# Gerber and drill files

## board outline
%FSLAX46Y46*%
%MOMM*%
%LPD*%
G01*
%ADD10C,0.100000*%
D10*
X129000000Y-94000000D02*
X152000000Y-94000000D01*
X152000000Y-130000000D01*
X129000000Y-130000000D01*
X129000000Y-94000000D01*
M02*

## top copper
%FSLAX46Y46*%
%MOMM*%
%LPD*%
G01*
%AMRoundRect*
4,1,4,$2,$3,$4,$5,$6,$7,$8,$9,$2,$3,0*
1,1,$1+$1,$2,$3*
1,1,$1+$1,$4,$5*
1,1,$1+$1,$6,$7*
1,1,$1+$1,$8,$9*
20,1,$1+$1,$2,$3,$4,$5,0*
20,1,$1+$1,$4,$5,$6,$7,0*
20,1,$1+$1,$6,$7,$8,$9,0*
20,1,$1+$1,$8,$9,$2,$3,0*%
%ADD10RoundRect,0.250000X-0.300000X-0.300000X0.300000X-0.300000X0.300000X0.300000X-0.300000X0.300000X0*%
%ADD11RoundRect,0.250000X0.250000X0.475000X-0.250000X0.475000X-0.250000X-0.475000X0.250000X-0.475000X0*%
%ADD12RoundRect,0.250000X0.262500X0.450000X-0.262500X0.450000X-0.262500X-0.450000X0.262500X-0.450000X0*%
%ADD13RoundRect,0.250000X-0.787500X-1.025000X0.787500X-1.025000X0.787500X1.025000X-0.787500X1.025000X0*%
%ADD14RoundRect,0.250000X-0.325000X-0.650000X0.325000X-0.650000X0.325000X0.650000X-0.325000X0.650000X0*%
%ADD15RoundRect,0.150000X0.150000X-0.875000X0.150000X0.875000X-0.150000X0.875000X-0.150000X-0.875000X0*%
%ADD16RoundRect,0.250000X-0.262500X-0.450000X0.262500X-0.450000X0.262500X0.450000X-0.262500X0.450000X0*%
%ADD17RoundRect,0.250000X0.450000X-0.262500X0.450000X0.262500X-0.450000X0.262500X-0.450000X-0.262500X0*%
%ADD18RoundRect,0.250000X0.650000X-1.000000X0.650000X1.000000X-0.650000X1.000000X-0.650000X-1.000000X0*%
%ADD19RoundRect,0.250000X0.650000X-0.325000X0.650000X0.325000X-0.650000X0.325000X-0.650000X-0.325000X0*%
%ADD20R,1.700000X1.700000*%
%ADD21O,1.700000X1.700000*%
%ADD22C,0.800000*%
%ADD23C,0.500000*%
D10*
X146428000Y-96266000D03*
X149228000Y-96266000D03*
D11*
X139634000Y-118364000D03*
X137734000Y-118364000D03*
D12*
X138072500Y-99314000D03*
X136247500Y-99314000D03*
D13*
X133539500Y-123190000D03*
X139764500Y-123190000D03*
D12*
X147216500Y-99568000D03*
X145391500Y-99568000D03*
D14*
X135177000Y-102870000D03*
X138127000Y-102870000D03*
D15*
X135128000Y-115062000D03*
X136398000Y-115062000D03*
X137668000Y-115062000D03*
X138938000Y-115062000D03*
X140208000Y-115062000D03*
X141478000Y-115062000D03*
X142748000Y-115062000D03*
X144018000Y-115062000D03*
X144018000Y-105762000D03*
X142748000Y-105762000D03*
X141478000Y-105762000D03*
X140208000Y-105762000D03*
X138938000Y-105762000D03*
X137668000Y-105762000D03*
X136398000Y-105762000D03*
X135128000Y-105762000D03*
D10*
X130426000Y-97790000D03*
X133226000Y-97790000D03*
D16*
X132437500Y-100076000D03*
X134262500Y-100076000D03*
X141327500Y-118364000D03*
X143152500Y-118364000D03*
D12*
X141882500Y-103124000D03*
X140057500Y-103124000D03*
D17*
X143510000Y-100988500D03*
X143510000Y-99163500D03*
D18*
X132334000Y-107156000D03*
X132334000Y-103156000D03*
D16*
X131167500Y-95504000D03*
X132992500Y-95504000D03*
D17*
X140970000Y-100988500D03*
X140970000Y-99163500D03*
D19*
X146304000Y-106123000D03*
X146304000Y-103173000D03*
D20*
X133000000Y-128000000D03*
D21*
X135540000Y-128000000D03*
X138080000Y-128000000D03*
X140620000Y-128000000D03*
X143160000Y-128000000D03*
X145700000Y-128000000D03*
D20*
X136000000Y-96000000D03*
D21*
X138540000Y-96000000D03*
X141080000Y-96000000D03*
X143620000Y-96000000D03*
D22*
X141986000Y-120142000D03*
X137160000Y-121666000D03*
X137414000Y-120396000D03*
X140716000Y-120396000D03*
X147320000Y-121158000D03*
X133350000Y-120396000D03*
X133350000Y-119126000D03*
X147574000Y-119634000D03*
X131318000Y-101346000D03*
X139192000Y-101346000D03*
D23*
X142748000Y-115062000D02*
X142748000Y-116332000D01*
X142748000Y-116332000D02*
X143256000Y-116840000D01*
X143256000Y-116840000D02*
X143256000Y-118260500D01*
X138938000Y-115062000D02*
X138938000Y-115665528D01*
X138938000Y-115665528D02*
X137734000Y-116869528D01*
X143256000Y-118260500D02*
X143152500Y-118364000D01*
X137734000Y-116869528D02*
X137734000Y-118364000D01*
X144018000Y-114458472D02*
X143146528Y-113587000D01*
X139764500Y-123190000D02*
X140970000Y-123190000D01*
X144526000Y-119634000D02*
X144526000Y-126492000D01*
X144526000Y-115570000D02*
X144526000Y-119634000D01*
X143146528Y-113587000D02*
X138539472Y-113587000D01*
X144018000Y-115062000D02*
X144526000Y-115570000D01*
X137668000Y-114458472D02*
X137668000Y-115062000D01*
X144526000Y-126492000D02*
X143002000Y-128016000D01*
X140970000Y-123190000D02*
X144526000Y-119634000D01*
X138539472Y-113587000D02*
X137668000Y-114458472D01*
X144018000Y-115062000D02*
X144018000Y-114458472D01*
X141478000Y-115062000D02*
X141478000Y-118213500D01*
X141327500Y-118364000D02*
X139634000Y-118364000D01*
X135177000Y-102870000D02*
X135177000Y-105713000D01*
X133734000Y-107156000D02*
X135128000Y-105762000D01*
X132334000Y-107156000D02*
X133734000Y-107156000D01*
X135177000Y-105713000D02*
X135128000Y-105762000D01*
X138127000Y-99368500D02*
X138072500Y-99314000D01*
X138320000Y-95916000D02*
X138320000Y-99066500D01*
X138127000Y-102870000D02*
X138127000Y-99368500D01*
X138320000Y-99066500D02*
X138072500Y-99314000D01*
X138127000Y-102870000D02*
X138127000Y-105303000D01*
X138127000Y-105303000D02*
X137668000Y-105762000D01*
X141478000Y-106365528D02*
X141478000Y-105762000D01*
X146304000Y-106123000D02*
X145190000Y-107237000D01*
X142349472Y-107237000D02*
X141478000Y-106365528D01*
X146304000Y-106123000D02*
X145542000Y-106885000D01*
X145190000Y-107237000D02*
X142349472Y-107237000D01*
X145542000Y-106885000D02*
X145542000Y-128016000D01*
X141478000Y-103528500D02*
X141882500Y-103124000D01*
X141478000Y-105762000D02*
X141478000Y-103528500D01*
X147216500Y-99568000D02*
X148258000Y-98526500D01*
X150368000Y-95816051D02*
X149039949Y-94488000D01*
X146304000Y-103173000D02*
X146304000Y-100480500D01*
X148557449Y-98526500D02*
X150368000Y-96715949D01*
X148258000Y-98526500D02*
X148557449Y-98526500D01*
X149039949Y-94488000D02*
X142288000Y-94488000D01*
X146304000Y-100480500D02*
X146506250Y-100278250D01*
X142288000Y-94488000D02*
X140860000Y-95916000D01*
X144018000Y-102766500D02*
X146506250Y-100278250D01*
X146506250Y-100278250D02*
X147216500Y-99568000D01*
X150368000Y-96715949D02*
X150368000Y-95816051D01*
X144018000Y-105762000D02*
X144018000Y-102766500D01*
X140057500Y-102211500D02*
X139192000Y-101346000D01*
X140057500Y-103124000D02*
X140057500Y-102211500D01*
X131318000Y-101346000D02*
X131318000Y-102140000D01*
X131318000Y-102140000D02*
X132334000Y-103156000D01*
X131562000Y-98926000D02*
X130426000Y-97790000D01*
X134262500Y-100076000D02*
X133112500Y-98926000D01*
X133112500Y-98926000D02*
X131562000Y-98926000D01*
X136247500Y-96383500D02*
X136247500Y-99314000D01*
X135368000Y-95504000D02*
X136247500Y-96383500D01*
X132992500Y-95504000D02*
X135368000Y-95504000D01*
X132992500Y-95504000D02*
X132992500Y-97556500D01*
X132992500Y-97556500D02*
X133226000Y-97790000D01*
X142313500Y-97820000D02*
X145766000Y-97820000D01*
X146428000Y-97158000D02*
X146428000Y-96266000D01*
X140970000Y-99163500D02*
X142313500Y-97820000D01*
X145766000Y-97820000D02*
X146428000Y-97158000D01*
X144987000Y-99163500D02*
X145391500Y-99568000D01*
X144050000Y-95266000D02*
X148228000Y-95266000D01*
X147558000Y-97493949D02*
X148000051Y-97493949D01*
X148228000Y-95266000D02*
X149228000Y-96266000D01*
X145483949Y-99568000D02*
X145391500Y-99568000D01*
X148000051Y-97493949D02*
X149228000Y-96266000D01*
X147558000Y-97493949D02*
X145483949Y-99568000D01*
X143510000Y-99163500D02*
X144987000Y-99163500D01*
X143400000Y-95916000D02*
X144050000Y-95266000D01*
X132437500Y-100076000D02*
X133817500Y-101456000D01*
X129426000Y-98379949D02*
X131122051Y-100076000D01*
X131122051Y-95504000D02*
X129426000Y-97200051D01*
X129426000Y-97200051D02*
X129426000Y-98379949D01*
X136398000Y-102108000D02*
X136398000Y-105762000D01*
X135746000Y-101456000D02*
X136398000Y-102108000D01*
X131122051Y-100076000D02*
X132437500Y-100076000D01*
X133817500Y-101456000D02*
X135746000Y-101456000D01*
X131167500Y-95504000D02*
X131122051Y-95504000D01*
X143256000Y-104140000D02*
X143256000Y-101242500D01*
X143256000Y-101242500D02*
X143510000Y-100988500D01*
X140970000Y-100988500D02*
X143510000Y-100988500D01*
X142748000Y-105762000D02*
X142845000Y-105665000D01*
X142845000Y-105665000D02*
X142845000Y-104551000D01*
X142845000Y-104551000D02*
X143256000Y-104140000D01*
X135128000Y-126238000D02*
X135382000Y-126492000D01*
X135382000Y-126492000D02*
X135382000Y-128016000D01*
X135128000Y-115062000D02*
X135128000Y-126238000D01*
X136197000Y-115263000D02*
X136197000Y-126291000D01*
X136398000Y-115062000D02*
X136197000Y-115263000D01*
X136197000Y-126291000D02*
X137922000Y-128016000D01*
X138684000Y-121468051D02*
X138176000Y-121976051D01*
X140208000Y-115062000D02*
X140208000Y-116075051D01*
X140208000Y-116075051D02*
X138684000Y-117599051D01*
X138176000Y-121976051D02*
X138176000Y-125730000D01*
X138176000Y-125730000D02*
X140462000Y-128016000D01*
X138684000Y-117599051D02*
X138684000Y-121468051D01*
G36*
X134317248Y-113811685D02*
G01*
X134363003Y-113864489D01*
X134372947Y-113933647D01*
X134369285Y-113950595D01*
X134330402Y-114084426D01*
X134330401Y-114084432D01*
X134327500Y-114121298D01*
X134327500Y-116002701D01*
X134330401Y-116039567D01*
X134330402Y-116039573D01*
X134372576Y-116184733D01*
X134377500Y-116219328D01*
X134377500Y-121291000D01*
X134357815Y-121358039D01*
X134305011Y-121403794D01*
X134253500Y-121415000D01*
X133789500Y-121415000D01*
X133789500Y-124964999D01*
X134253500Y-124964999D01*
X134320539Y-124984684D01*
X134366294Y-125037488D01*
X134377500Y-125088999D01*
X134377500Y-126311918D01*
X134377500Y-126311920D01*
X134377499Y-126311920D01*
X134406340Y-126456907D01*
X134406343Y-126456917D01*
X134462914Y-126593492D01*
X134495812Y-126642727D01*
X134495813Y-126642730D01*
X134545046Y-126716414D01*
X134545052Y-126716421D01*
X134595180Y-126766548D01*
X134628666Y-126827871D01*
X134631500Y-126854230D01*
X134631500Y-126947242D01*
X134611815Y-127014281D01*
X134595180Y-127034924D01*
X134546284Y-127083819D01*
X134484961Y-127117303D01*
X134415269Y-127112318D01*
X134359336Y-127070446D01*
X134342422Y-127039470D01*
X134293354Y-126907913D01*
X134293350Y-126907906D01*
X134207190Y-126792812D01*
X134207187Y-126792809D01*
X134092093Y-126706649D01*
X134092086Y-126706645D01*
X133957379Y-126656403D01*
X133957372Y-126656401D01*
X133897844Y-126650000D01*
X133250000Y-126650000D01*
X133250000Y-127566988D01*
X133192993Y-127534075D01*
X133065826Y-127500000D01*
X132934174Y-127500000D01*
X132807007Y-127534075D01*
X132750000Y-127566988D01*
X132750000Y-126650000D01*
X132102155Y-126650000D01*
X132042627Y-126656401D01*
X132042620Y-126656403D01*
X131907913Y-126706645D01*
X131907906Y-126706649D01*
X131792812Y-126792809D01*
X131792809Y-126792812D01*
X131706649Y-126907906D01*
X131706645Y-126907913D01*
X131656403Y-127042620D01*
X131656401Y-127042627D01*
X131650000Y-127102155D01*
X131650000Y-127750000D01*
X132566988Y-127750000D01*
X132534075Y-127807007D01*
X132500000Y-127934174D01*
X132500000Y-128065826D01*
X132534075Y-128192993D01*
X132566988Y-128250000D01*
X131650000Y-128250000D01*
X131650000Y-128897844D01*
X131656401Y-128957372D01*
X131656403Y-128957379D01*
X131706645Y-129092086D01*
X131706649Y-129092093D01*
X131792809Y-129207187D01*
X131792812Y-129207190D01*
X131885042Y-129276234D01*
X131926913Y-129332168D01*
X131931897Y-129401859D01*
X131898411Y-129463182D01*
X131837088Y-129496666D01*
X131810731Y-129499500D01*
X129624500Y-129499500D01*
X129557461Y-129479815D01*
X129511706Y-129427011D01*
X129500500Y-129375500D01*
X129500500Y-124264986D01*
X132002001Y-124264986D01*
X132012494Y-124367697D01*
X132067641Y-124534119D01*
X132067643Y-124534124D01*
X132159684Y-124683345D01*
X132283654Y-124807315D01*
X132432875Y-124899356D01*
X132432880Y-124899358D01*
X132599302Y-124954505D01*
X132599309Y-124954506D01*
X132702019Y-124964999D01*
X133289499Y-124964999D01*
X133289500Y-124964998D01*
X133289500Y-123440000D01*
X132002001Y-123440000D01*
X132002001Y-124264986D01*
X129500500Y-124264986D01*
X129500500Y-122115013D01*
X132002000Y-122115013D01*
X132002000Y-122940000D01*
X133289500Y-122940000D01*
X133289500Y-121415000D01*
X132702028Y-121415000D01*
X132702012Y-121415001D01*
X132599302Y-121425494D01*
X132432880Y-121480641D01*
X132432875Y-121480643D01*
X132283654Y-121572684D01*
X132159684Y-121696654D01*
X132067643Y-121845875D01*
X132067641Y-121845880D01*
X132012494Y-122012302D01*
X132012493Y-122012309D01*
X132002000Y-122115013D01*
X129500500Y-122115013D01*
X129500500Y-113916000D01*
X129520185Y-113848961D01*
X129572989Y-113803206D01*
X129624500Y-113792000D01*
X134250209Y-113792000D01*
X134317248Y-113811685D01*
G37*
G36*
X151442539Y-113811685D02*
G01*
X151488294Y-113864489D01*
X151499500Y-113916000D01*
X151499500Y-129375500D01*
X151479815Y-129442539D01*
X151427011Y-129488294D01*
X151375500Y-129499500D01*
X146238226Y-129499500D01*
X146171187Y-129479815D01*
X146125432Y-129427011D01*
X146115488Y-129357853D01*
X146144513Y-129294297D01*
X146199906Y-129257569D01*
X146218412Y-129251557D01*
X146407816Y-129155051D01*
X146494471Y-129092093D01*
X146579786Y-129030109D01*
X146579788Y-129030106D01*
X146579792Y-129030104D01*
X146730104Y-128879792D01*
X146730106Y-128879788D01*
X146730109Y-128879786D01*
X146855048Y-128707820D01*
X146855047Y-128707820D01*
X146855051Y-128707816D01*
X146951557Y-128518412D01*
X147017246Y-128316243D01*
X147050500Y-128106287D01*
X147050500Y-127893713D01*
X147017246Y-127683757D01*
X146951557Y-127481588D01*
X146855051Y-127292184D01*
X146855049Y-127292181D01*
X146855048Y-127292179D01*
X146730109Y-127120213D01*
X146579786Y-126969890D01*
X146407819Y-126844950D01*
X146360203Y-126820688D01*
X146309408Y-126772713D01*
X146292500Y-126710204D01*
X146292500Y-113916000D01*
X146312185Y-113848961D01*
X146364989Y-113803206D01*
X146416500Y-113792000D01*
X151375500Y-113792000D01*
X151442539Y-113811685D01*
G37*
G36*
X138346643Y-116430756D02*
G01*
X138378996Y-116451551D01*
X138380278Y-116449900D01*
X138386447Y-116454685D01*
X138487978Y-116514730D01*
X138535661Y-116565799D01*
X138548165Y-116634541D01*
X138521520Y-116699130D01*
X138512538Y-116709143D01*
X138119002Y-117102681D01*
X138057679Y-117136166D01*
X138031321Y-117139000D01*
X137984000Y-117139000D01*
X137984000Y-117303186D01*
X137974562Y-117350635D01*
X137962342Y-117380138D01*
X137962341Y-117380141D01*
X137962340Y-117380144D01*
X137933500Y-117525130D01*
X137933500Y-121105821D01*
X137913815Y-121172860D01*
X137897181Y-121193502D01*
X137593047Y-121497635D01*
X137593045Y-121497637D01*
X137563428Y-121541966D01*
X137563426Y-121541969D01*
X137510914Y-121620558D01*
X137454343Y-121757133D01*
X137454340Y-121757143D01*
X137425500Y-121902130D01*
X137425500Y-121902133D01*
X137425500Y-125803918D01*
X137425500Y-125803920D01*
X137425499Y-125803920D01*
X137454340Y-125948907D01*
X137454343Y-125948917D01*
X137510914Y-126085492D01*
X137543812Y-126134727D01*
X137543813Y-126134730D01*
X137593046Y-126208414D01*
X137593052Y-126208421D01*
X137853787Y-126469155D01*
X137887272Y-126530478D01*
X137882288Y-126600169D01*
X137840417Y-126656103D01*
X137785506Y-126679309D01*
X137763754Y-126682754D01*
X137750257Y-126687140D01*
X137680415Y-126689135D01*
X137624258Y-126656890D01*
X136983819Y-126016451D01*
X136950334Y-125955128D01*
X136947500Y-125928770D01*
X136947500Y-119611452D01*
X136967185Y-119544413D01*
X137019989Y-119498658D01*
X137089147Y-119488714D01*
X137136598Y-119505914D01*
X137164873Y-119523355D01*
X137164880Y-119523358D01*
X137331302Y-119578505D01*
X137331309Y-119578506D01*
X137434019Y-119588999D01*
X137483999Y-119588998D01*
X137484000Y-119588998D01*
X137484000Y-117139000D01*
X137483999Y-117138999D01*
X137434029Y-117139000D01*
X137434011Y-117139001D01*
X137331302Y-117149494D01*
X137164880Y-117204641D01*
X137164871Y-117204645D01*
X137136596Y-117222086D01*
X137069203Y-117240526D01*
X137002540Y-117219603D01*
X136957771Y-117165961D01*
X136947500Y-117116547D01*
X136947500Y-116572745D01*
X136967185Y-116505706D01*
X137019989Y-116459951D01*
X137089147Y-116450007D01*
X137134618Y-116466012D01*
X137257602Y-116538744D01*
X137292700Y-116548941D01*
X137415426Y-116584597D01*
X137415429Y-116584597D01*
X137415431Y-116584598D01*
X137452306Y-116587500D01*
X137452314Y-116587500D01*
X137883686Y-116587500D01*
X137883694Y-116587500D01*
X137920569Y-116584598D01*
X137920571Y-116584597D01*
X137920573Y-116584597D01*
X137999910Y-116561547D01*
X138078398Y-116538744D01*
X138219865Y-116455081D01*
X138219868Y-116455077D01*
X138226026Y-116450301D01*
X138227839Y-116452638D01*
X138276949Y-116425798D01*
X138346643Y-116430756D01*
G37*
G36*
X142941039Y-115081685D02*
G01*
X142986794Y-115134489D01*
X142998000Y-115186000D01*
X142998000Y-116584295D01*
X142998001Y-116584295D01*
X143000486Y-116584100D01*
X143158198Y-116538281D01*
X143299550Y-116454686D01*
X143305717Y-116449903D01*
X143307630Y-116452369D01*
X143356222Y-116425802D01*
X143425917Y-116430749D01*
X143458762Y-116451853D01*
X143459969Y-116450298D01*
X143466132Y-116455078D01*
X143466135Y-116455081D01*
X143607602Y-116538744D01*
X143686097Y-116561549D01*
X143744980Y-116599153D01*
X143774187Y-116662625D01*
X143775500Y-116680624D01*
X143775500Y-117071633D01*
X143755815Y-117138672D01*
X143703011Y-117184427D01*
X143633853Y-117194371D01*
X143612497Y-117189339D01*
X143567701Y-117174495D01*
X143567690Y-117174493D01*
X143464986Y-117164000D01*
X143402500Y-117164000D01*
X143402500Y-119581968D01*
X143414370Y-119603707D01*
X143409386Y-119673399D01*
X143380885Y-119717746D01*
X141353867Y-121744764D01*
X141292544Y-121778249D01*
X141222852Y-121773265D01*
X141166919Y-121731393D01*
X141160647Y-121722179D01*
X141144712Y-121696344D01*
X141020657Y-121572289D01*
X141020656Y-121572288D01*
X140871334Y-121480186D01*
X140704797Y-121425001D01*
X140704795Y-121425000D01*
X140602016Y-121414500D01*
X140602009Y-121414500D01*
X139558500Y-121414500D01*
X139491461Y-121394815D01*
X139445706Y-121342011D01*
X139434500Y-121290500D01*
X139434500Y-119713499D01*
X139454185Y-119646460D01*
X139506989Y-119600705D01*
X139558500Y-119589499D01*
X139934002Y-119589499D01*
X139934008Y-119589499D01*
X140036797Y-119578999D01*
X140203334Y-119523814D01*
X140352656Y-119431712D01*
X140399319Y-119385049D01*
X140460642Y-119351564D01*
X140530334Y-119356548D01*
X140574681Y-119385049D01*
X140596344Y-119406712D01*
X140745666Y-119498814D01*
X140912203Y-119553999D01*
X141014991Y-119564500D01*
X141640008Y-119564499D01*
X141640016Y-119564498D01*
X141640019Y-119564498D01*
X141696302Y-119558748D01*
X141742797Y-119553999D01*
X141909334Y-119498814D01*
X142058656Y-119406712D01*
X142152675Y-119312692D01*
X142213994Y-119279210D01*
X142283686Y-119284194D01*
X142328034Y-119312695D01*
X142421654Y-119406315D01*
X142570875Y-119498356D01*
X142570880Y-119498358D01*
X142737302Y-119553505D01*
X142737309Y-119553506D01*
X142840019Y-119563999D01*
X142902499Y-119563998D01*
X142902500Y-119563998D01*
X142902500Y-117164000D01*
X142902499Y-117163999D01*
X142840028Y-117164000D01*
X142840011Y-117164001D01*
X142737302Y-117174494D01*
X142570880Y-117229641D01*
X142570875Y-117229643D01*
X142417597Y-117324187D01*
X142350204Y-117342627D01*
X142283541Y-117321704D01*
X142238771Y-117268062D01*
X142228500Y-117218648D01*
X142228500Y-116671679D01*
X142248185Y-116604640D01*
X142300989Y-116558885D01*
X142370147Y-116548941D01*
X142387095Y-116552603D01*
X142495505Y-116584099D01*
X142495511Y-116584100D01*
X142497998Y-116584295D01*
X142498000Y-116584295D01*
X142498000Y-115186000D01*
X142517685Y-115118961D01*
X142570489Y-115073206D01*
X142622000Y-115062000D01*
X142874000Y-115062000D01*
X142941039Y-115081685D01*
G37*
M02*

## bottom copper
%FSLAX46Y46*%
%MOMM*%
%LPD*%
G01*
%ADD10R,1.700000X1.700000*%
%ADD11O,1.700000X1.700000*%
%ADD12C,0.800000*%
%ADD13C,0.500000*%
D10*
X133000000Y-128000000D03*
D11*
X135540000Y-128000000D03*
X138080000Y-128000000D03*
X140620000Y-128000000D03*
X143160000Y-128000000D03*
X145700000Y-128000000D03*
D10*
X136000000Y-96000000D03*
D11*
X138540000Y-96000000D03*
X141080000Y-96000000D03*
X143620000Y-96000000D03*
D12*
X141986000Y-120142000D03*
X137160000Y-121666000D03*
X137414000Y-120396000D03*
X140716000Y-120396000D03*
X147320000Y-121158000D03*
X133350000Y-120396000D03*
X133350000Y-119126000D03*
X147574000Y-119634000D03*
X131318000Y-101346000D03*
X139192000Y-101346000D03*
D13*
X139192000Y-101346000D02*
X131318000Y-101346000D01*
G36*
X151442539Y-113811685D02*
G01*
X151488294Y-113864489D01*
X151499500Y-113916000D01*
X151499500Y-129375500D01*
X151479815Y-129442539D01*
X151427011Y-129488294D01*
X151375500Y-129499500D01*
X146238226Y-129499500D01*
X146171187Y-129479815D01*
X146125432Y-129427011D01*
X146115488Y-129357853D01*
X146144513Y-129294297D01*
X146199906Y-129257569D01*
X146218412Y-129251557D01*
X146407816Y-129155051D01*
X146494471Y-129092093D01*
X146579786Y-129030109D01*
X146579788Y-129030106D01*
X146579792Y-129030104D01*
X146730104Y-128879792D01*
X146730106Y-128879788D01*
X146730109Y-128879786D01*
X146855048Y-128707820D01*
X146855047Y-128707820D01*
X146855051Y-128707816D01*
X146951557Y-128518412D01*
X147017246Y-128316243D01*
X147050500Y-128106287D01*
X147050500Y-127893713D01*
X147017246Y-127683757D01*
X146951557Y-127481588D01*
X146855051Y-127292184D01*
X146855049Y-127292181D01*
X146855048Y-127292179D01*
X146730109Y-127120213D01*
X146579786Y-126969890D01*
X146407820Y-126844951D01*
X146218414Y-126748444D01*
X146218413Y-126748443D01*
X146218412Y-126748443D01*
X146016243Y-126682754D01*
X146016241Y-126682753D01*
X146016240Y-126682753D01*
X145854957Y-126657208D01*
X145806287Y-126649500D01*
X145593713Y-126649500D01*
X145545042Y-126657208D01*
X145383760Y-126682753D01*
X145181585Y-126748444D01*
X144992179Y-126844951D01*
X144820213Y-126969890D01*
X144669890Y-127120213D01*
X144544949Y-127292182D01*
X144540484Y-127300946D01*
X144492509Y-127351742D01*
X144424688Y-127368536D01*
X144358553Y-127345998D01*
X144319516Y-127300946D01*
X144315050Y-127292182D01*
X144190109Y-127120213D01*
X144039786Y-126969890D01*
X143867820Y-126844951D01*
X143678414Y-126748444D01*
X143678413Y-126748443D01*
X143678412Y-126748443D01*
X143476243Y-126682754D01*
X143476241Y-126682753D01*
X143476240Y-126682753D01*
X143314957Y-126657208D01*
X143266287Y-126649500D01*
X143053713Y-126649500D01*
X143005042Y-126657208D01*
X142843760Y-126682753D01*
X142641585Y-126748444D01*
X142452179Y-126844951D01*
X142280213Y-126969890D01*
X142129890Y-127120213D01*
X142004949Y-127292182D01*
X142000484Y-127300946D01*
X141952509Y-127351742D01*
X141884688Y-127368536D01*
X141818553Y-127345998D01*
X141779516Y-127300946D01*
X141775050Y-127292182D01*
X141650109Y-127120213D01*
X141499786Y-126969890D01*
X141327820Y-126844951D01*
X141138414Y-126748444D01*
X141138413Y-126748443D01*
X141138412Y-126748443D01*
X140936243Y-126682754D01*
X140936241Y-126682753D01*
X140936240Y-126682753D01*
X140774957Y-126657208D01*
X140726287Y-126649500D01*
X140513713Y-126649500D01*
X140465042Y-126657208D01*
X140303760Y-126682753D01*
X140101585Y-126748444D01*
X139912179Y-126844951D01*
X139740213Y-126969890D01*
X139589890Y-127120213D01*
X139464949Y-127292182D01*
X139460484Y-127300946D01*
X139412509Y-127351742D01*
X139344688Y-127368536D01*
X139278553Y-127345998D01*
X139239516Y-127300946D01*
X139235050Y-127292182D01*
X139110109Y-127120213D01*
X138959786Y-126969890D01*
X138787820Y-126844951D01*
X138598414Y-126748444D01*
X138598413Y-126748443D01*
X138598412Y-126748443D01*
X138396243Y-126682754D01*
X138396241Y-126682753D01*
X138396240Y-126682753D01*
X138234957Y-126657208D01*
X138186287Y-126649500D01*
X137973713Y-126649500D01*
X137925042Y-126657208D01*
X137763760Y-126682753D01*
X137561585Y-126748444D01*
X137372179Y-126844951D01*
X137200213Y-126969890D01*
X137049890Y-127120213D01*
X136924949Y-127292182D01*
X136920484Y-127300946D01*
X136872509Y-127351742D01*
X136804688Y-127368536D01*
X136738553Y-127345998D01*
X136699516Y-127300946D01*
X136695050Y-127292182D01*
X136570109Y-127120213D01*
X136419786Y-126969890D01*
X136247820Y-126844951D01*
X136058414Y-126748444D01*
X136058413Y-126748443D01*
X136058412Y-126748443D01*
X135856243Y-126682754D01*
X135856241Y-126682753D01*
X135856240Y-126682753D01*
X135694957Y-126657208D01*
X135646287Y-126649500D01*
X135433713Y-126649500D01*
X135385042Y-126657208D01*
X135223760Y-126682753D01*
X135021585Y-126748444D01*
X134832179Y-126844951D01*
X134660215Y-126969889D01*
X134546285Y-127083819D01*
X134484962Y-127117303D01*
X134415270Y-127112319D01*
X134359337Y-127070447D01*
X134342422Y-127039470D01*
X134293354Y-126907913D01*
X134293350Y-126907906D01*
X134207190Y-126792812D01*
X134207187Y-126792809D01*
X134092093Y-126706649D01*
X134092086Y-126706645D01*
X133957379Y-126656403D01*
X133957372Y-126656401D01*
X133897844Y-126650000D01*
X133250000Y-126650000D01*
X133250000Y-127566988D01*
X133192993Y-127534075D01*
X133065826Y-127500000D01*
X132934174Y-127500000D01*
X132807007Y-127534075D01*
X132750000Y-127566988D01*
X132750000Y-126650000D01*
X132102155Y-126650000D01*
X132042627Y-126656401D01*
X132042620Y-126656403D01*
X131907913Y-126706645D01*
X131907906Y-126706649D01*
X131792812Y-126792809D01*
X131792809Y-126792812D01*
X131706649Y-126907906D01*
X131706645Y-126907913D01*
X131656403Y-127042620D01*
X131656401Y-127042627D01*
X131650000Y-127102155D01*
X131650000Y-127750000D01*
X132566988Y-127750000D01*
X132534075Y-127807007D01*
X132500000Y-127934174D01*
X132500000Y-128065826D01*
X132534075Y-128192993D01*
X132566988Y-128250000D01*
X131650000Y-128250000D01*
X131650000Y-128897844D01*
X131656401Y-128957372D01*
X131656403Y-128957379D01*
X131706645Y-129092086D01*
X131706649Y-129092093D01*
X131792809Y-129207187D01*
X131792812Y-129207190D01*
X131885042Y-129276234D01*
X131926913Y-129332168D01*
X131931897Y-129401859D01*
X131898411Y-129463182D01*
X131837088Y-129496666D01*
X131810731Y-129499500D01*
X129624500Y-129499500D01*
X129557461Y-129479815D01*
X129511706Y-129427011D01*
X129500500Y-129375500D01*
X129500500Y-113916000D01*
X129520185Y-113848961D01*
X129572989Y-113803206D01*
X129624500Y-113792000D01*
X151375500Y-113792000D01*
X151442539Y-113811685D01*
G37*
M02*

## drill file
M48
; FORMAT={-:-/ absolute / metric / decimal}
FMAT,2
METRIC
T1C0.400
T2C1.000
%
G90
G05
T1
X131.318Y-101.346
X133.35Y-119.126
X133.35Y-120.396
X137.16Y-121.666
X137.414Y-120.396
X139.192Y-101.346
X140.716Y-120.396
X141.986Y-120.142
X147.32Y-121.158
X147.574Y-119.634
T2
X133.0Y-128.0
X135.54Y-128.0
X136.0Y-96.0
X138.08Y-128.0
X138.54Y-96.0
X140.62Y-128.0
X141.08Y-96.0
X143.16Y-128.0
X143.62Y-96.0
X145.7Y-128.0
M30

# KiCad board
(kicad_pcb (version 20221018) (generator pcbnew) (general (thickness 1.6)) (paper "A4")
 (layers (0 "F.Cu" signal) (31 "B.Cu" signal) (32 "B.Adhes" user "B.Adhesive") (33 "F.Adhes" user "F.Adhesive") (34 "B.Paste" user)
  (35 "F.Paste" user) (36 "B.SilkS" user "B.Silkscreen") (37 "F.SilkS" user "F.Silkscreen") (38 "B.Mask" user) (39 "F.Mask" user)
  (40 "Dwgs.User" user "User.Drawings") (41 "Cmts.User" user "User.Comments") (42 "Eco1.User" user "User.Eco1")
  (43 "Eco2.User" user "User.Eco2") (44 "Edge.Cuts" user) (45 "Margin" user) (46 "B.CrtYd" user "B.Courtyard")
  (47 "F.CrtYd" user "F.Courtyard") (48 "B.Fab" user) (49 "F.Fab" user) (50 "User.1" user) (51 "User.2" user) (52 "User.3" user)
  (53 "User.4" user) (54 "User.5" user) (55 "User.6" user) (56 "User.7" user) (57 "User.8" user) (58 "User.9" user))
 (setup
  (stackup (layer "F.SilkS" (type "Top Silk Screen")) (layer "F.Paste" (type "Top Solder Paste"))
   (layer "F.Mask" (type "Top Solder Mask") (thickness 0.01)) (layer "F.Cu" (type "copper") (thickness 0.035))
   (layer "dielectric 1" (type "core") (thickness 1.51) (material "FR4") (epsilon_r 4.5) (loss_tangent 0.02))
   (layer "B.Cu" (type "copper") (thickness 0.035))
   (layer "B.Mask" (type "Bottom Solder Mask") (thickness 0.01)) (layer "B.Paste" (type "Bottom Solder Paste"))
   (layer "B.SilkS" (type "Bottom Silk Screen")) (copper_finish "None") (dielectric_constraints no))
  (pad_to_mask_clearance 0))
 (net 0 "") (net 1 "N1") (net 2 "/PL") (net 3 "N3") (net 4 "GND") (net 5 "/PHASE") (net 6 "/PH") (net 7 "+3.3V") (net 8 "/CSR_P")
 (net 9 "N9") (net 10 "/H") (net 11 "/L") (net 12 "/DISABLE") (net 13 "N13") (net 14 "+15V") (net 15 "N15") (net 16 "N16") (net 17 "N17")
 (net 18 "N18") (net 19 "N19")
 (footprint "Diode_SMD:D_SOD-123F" (layer "F.Cu") (at 147.828 96.266)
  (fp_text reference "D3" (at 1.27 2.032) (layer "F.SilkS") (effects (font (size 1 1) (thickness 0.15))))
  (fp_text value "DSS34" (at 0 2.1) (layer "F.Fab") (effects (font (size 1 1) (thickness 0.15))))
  (pad "1" smd roundrect (at -1.4 0) (size 1.1 1.1) (layers "F.Cu" "F.Paste" "F.Mask") (roundrect_rratio 0.2272727273) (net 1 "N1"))
  (pad "2" smd roundrect (at 1.4 0) (size 1.1 1.1) (layers "F.Cu" "F.Paste" "F.Mask") (roundrect_rratio 0.2272727273) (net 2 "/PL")))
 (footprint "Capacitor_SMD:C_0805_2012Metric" (layer "F.Cu") (at 138.684 118.364 180)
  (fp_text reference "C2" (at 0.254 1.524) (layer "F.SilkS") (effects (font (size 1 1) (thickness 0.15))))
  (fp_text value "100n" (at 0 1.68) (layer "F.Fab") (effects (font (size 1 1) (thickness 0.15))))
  (pad "1" smd roundrect (at -0.95 0 180) (size 1 1.45) (layers "F.Cu" "F.Paste" "F.Mask") (roundrect_rratio 0.25) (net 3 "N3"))
  (pad "2" smd roundrect (at 0.95 0 180) (size 1 1.45) (layers "F.Cu" "F.Paste" "F.Mask") (roundrect_rratio 0.25) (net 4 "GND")))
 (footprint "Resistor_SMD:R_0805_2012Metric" (layer "F.Cu") (at 137.16 99.314 180)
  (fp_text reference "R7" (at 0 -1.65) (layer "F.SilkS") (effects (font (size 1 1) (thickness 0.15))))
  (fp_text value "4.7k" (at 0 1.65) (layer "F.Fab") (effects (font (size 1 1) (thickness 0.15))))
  (pad "1" smd roundrect (at -0.9125 0 180) (size 1.025 1.4) (layers "F.Cu" "F.Paste" "F.Mask") (roundrect_rratio 0.243902) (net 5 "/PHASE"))
  (pad "2" smd roundrect (at 0.9125 0 180) (size 1.025 1.4) (layers "F.Cu" "F.Paste" "F.Mask") (roundrect_rratio 0.243902) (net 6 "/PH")))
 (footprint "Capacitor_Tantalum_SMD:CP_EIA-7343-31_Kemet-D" (layer "F.Cu") (at 136.652 123.19)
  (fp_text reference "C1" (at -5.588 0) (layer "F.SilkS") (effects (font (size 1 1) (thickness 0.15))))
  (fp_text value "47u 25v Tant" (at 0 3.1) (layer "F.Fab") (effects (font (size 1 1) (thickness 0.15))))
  (pad "1" smd roundrect (at -3.1125 0) (size 2.075 2.55) (layers "F.Cu" "F.Paste" "F.Mask") (roundrect_rratio 0.120482) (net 4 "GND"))
  (pad "2" smd roundrect (at 3.1125 0) (size 2.075 2.55) (layers "F.Cu" "F.Paste" "F.Mask") (roundrect_rratio 0.120482) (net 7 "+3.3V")))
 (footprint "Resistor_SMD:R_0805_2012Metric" (layer "F.Cu") (at 146.304 99.568 180)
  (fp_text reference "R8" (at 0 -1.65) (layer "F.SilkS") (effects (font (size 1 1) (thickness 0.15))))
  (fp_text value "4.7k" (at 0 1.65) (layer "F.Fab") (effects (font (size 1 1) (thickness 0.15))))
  (pad "1" smd roundrect (at -0.9125 0 180) (size 1.025 1.4) (layers "F.Cu" "F.Paste" "F.Mask") (roundrect_rratio 0.243902) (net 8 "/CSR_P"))
  (pad "2" smd roundrect (at 0.9125 0 180) (size 1.025 1.4) (layers "F.Cu" "F.Paste" "F.Mask") (roundrect_rratio 0.243902) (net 2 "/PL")))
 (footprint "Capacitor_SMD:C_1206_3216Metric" (layer "F.Cu") (at 136.652 102.87)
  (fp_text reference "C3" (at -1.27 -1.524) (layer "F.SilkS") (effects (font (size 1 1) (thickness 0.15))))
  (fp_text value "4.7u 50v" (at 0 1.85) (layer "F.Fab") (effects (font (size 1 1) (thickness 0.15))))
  (pad "1" smd roundrect (at -1.475 0) (size 1.15 1.8) (layers "F.Cu" "F.Paste" "F.Mask") (roundrect_rratio 0.217391) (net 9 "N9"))
  (pad "2" smd roundrect (at 1.475 0) (size 1.15 1.8) (layers "F.Cu" "F.Paste" "F.Mask") (roundrect_rratio 0.217391) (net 5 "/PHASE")))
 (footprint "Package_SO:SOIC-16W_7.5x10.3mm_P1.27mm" (layer "F.Cu") (at 139.573 110.412 90)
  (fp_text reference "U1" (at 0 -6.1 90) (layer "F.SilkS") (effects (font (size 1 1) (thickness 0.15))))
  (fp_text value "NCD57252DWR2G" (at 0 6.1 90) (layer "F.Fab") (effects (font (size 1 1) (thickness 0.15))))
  (pad "1" smd roundrect (at -4.65 -4.445 90) (size 2.05 0.6) (layers "F.Cu" "F.Paste" "F.Mask") (roundrect_rratio 0.25) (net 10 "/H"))
  (pad "2" smd roundrect (at -4.65 -3.175 90) (size 2.05 0.6) (layers "F.Cu" "F.Paste" "F.Mask") (roundrect_rratio 0.25) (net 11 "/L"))
  (pad "3" smd roundrect (at -4.65 -1.905 90) (size 2.05 0.6) (layers "F.Cu" "F.Paste" "F.Mask") (roundrect_rratio 0.25) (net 7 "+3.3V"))
  (pad "4" smd roundrect (at -4.65 -0.635 90) (size 2.05 0.6) (layers "F.Cu" "F.Paste" "F.Mask") (roundrect_rratio 0.25) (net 4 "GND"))
  (pad "5" smd roundrect (at -4.65 0.635 90) (size 2.05 0.6) (layers "F.Cu" "F.Paste" "F.Mask") (roundrect_rratio 0.25) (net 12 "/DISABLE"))
  (pad "6" smd roundrect (at -4.65 1.905 90) (size 2.05 0.6) (layers "F.Cu" "F.Paste" "F.Mask") (roundrect_rratio 0.25) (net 3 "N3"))
  (pad "7" smd roundrect (at -4.65 3.175 90) (size 2.05 0.6) (layers "F.Cu" "F.Paste" "F.Mask") (roundrect_rratio 0.25) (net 4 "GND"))
  (pad "8" smd roundrect (at -4.65 4.445 90) (size 2.05 0.6) (layers "F.Cu" "F.Paste" "F.Mask") (roundrect_rratio 0.25) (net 7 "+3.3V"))
  (pad "9" smd roundrect (at 4.65 4.445 90) (size 2.05 0.6) (layers "F.Cu" "F.Paste" "F.Mask") (roundrect_rratio 0.25) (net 8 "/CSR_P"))
  (pad "10" smd roundrect (at 4.65 3.175 90) (size 2.05 0.6) (layers "F.Cu" "F.Paste" "F.Mask") (roundrect_rratio 0.25) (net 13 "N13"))
  (pad "11" smd roundrect (at 4.65 1.905 90) (size 2.05 0.6) (layers "F.Cu" "F.Paste" "F.Mask") (roundrect_rratio 0.25) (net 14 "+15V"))
  (pad "12" smd roundrect (at 4.65 0.635 90) (size 2.05 0.6) (layers "F.Cu" "F.Paste" "F.Mask") (roundrect_rratio 0.25) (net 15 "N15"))
  (pad "13" smd roundrect (at 4.65 -0.635 90) (size 2.05 0.6) (layers "F.Cu" "F.Paste" "F.Mask") (roundrect_rratio 0.25) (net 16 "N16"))
  (pad "14" smd roundrect (at 4.65 -1.905 90) (size 2.05 0.6) (layers "F.Cu" "F.Paste" "F.Mask") (roundrect_rratio 0.25) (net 5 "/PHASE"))
  (pad "15" smd roundrect (at 4.65 -3.175 90) (size 2.05 0.6) (layers "F.Cu" "F.Paste" "F.Mask") (roundrect_rratio 0.25) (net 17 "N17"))
  (pad "16" smd roundrect (at 4.65 -4.445 90) (size 2.05 0.6) (layers "F.Cu" "F.Paste" "F.Mask") (roundrect_rratio 0.25) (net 9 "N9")))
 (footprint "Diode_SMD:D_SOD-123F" (layer "F.Cu") (at 131.826 97.79)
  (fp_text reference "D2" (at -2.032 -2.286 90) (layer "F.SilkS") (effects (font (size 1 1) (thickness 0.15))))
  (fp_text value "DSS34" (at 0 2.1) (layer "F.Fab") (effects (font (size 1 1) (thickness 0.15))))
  (pad "1" smd roundrect (at -1.4 0) (size 1.1 1.1) (layers "F.Cu" "F.Paste" "F.Mask") (roundrect_rratio 0.2272727273) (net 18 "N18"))
  (pad "2" smd roundrect (at 1.4 0) (size 1.1 1.1) (layers "F.Cu" "F.Paste" "F.Mask") (roundrect_rratio 0.2272727273) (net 6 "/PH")))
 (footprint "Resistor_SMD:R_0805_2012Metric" (layer "F.Cu") (at 133.35 100.076)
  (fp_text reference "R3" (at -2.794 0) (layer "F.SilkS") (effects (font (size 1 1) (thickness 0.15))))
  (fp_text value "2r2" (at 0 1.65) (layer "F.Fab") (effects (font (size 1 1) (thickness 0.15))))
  (pad "1" smd roundrect (at -0.9125 0) (size 1.025 1.4) (layers "F.Cu" "F.Paste" "F.Mask") (roundrect_rratio 0.243902) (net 17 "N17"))
  (pad "2" smd roundrect (at 0.9125 0) (size 1.025 1.4) (layers "F.Cu" "F.Paste" "F.Mask") (roundrect_rratio 0.243902) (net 18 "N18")))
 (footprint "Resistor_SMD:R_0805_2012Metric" (layer "F.Cu") (at 142.24 118.364)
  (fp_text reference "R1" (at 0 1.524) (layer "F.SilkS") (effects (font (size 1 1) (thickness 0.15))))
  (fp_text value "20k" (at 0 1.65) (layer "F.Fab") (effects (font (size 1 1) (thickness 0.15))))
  (pad "1" smd roundrect (at -0.9125 0) (size 1.025 1.4) (layers "F.Cu" "F.Paste" "F.Mask") (roundrect_rratio 0.243902) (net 3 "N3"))
  (pad "2" smd roundrect (at 0.9125 0) (size 1.025 1.4) (layers "F.Cu" "F.Paste" "F.Mask") (roundrect_rratio 0.243902) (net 4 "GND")))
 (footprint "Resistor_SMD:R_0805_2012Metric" (layer "F.Cu") (at 140.97 103.124 180)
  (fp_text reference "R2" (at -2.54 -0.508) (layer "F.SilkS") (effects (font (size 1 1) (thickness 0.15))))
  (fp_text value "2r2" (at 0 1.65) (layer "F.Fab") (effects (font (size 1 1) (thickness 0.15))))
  (pad "1" smd roundrect (at -0.9125 0 180) (size 1.025 1.4) (layers "F.Cu" "F.Paste" "F.Mask") (roundrect_rratio 0.243902) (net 14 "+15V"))
  (pad "2" smd roundrect (at 0.9125 0 180) (size 1.025 1.4) (layers "F.Cu" "F.Paste" "F.Mask") (roundrect_rratio 0.243902) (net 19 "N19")))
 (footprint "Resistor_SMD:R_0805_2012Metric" (layer "F.Cu") (at 143.51 100.076 90)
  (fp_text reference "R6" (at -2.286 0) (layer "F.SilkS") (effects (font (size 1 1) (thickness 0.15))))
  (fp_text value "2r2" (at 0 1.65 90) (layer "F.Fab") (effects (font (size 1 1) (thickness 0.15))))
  (pad "1" smd roundrect (at -0.9125 0 90) (size 1.025 1.4) (layers "F.Cu" "F.Paste" "F.Mask") (roundrect_rratio 0.243902) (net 13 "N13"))
  (pad "2" smd roundrect (at 0.9125 0 90) (size 1.025 1.4) (layers "F.Cu" "F.Paste" "F.Mask") (roundrect_rratio 0.243902) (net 2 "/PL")))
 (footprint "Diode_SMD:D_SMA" (layer "F.Cu") (at 132.334 105.156 90)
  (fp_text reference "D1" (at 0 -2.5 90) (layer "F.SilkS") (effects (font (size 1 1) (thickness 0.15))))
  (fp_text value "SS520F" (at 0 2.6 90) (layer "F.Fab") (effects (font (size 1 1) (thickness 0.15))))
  (pad "1" smd roundrect (at -2 0 90) (size 2.5 1.8) (layers "F.Cu" "F.Paste" "F.Mask") (roundrect_rratio 0.1388888889) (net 9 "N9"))
  (pad "2" smd roundrect (at 2 0 90) (size 2.5 1.8) (layers "F.Cu" "F.Paste" "F.Mask") (roundrect_rratio 0.1388888889) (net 19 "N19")))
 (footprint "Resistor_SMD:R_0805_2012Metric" (layer "F.Cu") (at 132.08 95.504)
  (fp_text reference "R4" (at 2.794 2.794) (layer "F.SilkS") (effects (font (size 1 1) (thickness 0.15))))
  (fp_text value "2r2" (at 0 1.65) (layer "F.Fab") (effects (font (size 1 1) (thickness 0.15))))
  (pad "1" smd roundrect (at -0.9125 0) (size 1.025 1.4) (layers "F.Cu" "F.Paste" "F.Mask") (roundrect_rratio 0.243902) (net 17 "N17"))
  (pad "2" smd roundrect (at 0.9125 0) (size 1.025 1.4) (layers "F.Cu" "F.Paste" "F.Mask") (roundrect_rratio 0.243902) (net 6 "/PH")))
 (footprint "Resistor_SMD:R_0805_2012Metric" (layer "F.Cu") (at 140.97 100.076 90)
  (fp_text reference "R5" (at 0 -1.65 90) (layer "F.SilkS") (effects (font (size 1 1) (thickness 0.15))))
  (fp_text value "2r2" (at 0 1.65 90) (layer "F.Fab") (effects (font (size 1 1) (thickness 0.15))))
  (pad "1" smd roundrect (at -0.9125 0 90) (size 1.025 1.4) (layers "F.Cu" "F.Paste" "F.Mask") (roundrect_rratio 0.243902) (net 13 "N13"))
  (pad "2" smd roundrect (at 0.9125 0 90) (size 1.025 1.4) (layers "F.Cu" "F.Paste" "F.Mask") (roundrect_rratio 0.243902) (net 1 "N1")))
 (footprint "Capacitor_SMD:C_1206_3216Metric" (layer "F.Cu") (at 146.304 104.648 90)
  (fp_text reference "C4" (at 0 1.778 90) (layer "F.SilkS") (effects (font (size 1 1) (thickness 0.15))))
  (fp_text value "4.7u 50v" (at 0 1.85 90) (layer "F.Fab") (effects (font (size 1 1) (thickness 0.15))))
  (pad "1" smd roundrect (at -1.475 0 90) (size 1.15 1.8) (layers "F.Cu" "F.Paste" "F.Mask") (roundrect_rratio 0.217391) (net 14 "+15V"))
  (pad "2" smd roundrect (at 1.475 0 90) (size 1.15 1.8) (layers "F.Cu" "F.Paste" "F.Mask") (roundrect_rratio 0.217391) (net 8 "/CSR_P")))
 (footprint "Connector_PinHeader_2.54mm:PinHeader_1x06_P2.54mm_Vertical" (layer "B.Cu") (at 133 128 -90)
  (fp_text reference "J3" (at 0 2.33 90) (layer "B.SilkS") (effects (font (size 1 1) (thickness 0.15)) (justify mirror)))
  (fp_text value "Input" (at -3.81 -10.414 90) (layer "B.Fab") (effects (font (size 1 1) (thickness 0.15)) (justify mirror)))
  (pad "1" thru_hole rect (at 0 0 270) (size 1.7 1.7) (drill 1) (layers "*.Cu" "*.Mask") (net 4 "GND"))
  (pad "2" thru_hole oval (at 0 -2.54 270) (size 1.7 1.7) (drill 1) (layers "*.Cu" "*.Mask") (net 10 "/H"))
  (pad "3" thru_hole oval (at 0 -5.08 270) (size 1.7 1.7) (drill 1) (layers "*.Cu" "*.Mask") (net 11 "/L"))
  (pad "4" thru_hole oval (at 0 -7.62 270) (size 1.7 1.7) (drill 1) (layers "*.Cu" "*.Mask") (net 12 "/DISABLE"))
  (pad "5" thru_hole oval (at 0 -10.16 270) (size 1.7 1.7) (drill 1) (layers "*.Cu" "*.Mask") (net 7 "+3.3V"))
  (pad "6" thru_hole oval (at 0 -12.7 270) (size 1.7 1.7) (drill 1) (layers "*.Cu" "*.Mask") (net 14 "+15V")))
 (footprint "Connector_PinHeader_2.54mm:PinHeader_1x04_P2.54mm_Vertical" (layer "B.Cu") (at 136 96 -90)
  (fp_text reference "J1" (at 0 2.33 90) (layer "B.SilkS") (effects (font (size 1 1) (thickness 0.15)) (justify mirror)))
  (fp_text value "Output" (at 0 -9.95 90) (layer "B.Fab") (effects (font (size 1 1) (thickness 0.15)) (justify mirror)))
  (pad "1" thru_hole rect (at 0 0 270) (size 1.7 1.7) (drill 1) (layers "*.Cu" "*.Mask") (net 6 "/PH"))
  (pad "2" thru_hole oval (at 0 -2.54 270) (size 1.7 1.7) (drill 1) (layers "*.Cu" "*.Mask") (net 5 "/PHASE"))
  (pad "3" thru_hole oval (at 0 -5.08 270) (size 1.7 1.7) (drill 1) (layers "*.Cu" "*.Mask") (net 8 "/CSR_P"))
  (pad "4" thru_hole oval (at 0 -7.62 270) (size 1.7 1.7) (drill 1) (layers "*.Cu" "*.Mask") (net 2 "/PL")))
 (gr_rect (start 129 94) (end 152 130) (stroke (width 0.1) (type default)) (fill none) (layer "Edge.Cuts"))
 (segment (start 142.748 115.062) (end 142.748 116.332) (width 0.5) (layer "F.Cu") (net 4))
 (segment (start 142.748 116.332) (end 143.256 116.84) (width 0.5) (layer "F.Cu") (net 4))
 (segment (start 143.256 116.84) (end 143.256 118.2605) (width 0.5) (layer "F.Cu") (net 4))
 (segment (start 138.938 115.062) (end 138.938 115.665528) (width 0.5) (layer "F.Cu") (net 4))
 (segment (start 138.938 115.665528) (end 137.734 116.869528) (width 0.5) (layer "F.Cu") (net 4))
 (segment (start 143.256 118.2605) (end 143.1525 118.364) (width 0.5) (layer "F.Cu") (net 4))
 (segment (start 137.734 116.869528) (end 137.734 118.364) (width 0.5) (layer "F.Cu") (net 4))
 (via (at 141.986 120.142) (size 0.8) (drill 0.4) (layers "F.Cu" "B.Cu") (free) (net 4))
 (via (at 137.16 121.666) (size 0.8) (drill 0.4) (layers "F.Cu" "B.Cu") (free) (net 4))
 (via (at 137.414 120.396) (size 0.8) (drill 0.4) (layers "F.Cu" "B.Cu") (free) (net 4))
 (via (at 140.716 120.396) (size 0.8) (drill 0.4) (layers "F.Cu" "B.Cu") (free) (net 4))
 (via (at 147.32 121.158) (size 0.8) (drill 0.4) (layers "F.Cu" "B.Cu") (free) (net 4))
 (via (at 133.35 120.396) (size 0.8) (drill 0.4) (layers "F.Cu" "B.Cu") (free) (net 4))
 (via (at 133.35 119.126) (size 0.8) (drill 0.4) (layers "F.Cu" "B.Cu") (free) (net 4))
 (via (at 147.574 119.634) (size 0.8) (drill 0.4) (layers "F.Cu" "B.Cu") (free) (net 4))
 (segment (start 144.018 114.458472) (end 143.146528 113.587) (width 0.5) (layer "F.Cu") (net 7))
 (segment (start 139.7645 123.19) (end 140.97 123.19) (width 0.5) (layer "F.Cu") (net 7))
 (segment (start 144.526 119.634) (end 144.526 126.492) (width 0.5) (layer "F.Cu") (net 7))
 (segment (start 144.526 115.57) (end 144.526 119.634) (width 0.5) (layer "F.Cu") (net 7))
 (segment (start 143.146528 113.587) (end 138.539472 113.587) (width 0.5) (layer "F.Cu") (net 7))
 (segment (start 144.018 115.062) (end 144.526 115.57) (width 0.5) (layer "F.Cu") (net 7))
 (segment (start 137.668 114.458472) (end 137.668 115.062) (width 0.5) (layer "F.Cu") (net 7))
 (segment (start 144.526 126.492) (end 143.002 128.016) (width 0.5) (layer "F.Cu") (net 7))
 (segment (start 140.97 123.19) (end 144.526 119.634) (width 0.5) (layer "F.Cu") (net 7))
 (segment (start 138.539472 113.587) (end 137.668 114.458472) (width 0.5) (layer "F.Cu") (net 7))
 (segment (start 144.018 115.062) (end 144.018 114.458472) (width 0.5) (layer "F.Cu") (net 7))
 (segment (start 141.478 115.062) (end 141.478 118.2135) (width 0.5) (layer "F.Cu") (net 3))
 (segment (start 141.3275 118.364) (end 139.634 118.364) (width 0.5) (layer "F.Cu") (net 3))
 (segment (start 135.177 102.87) (end 135.177 105.713) (width 0.5) (layer "F.Cu") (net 9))
 (segment (start 133.734 107.156) (end 135.128 105.762) (width 0.5) (layer "F.Cu") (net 9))
 (segment (start 132.334 107.156) (end 133.734 107.156) (width 0.5) (layer "F.Cu") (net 9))
 (segment (start 135.177 105.713) (end 135.128 105.762) (width 0.5) (layer "F.Cu") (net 9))
 (segment (start 138.127 99.3685) (end 138.0725 99.314) (width 0.5) (layer "F.Cu") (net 5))
 (segment (start 138.32 95.916) (end 138.32 99.0665) (width 0.5) (layer "F.Cu") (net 5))
 (segment (start 138.127 102.87) (end 138.127 99.3685) (width 0.5) (layer "F.Cu") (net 5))
 (segment (start 138.32 99.0665) (end 138.0725 99.314) (width 0.5) (layer "F.Cu") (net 5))
 (segment (start 138.127 102.87) (end 138.127 105.303) (width 0.5) (layer "F.Cu") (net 5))
 (segment (start 138.127 105.303) (end 137.668 105.762) (width 0.5) (layer "F.Cu") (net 5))
 (segment (start 141.478 106.365528) (end 141.478 105.762) (width 0.5) (layer "F.Cu") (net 14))
 (segment (start 146.304 106.123) (end 145.19 107.237) (width 0.5) (layer "F.Cu") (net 14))
 (segment (start 142.349472 107.237) (end 141.478 106.365528) (width 0.5) (layer "F.Cu") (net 14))
 (segment (start 146.304 106.123) (end 145.542 106.885) (width 0.5) (layer "F.Cu") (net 14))
 (segment (start 145.19 107.237) (end 142.349472 107.237) (width 0.5) (layer "F.Cu") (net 14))
 (segment (start 145.542 106.885) (end 145.542 128.016) (width 0.5) (layer "F.Cu") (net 14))
 (segment (start 141.478 103.5285) (end 141.8825 103.124) (width 0.5) (layer "F.Cu") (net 14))
 (segment (start 141.478 105.762) (end 141.478 103.5285) (width 0.5) (layer "F.Cu") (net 14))
 (segment (start 147.2165 99.568) (end 148.258 98.5265) (width 0.5) (layer "F.Cu") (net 8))
 (segment (start 150.368 95.816051) (end 149.039949 94.488) (width 0.5) (layer "F.Cu") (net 8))
 (segment (start 146.304 103.173) (end 146.304 100.4805) (width 0.5) (layer "F.Cu") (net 8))
 (segment (start 148.557449 98.5265) (end 150.368 96.715949) (width 0.5) (layer "F.Cu") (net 8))
 (segment (start 148.258 98.5265) (end 148.557449 98.5265) (width 0.5) (layer "F.Cu") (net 8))
 (segment (start 149.039949 94.488) (end 142.288 94.488) (width 0.5) (layer "F.Cu") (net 8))
 (segment (start 146.304 100.4805) (end 146.50625 100.27825) (width 0.5) (layer "F.Cu") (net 8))
 (segment (start 142.288 94.488) (end 140.86 95.916) (width 0.5) (layer "F.Cu") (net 8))
 (segment (start 144.018 102.7665) (end 146.50625 100.27825) (width 0.5) (layer "F.Cu") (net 8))
 (segment (start 146.50625 100.27825) (end 147.2165 99.568) (width 0.5) (layer "F.Cu") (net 8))
 (segment (start 150.368 96.715949) (end 150.368 95.816051) (width 0.5) (layer "F.Cu") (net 8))
 (segment (start 144.018 105.762) (end 144.018 102.7665) (width 0.5) (layer "F.Cu") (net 8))
 (segment (start 140.0575 102.2115) (end 139.192 101.346) (width 0.5) (layer "F.Cu") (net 19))
 (segment (start 140.0575 103.124) (end 140.0575 102.2115) (width 0.5) (layer "F.Cu") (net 19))
 (segment (start 131.318 101.346) (end 131.318 102.14) (width 0.5) (layer "F.Cu") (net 19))
 (segment (start 131.318 102.14) (end 132.334 103.156) (width 0.5) (layer "F.Cu") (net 19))
 (via (at 131.318 101.346) (size 0.8) (drill 0.4) (layers "F.Cu" "B.Cu") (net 19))
 (via (at 139.192 101.346) (size 0.8) (drill 0.4) (layers "F.Cu" "B.Cu") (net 19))
 (segment (start 139.192 101.346) (end 131.318 101.346) (width 0.5) (layer "B.Cu") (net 19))
 (segment (start 131.562 98.926) (end 130.426 97.79) (width 0.5) (layer "F.Cu") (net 18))
 (segment (start 134.2625 100.076) (end 133.1125 98.926) (width 0.5) (layer "F.Cu") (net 18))
 (segment (start 133.1125 98.926) (end 131.562 98.926) (width 0.5) (layer "F.Cu") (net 18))
 (segment (start 136.2475 96.3835) (end 136.2475 99.314) (width 0.5) (layer "F.Cu") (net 6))
 (segment (start 135.368 95.504) (end 136.2475 96.3835) (width 0.5) (layer "F.Cu") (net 6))
 (segment (start 132.9925 95.504) (end 135.368 95.504) (width 0.5) (layer "F.Cu") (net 6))
 (segment (start 132.9925 95.504) (end 132.9925 97.5565) (width 0.5) (layer "F.Cu") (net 6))
 (segment (start 132.9925 97.5565) (end 133.226 97.79) (width 0.5) (layer "F.Cu") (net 6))
 (segment (start 142.3135 97.82) (end 145.766 97.82) (width 0.5) (layer "F.Cu") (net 1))
 (segment (start 146.428 97.158) (end 146.428 96.266) (width 0.5) (layer "F.Cu") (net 1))
 (segment (start 140.97 99.1635) (end 142.3135 97.82) (width 0.5) (layer "F.Cu") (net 1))
 (segment (start 145.766 97.82) (end 146.428 97.158) (width 0.5) (layer "F.Cu") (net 1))
 (segment (start 144.987 99.1635) (end 145.3915 99.568) (width 0.5) (layer "F.Cu") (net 2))
 (segment (start 144.05 95.266) (end 148.228 95.266) (width 0.5) (layer "F.Cu") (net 2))
 (segment (start 147.558 97.493949) (end 148.000051 97.493949) (width 0.5) (layer "F.Cu") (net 2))
 (segment (start 148.228 95.266) (end 149.228 96.266) (width 0.5) (layer "F.Cu") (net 2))
 (segment (start 145.483949 99.568) (end 145.3915 99.568) (width 0.5) (layer "F.Cu") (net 2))
 (segment (start 148.000051 97.493949) (end 149.228 96.266) (width 0.5) (layer "F.Cu") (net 2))
 (segment (start 147.558 97.493949) (end 145.483949 99.568) (width 0.5) (layer "F.Cu") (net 2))
 (segment (start 143.51 99.1635) (end 144.987 99.1635) (width 0.5) (layer "F.Cu") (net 2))
 (segment (start 143.4 95.916) (end 144.05 95.266) (width 0.5) (layer "F.Cu") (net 2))
 (segment (start 132.4375 100.076) (end 133.8175 101.456) (width 0.5) (layer "F.Cu") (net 17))
 (segment (start 129.426 98.379949) (end 131.122051 100.076) (width 0.5) (layer "F.Cu") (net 17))
 (segment (start 131.122051 95.504) (end 129.426 97.200051) (width 0.5) (layer "F.Cu") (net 17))
 (segment (start 129.426 97.200051) (end 129.426 98.379949) (width 0.5) (layer "F.Cu") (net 17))
 (segment (start 136.398 102.108) (end 136.398 105.762) (width 0.5) (layer "F.Cu") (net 17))
 (segment (start 135.746 101.456) (end 136.398 102.108) (width 0.5) (layer "F.Cu") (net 17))
 (segment (start 131.122051 100.076) (end 132.4375 100.076) (width 0.5) (layer "F.Cu") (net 17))
 (segment (start 133.8175 101.456) (end 135.746 101.456) (width 0.5) (layer "F.Cu") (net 17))
 (segment (start 131.1675 95.504) (end 131.122051 95.504) (width 0.5) (layer "F.Cu") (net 17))
 (segment (start 143.256 104.14) (end 143.256 101.2425) (width 0.5) (layer "F.Cu") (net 13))
 (segment (start 143.256 101.2425) (end 143.51 100.9885) (width 0.5) (layer "F.Cu") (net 13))
 (segment (start 140.97 100.9885) (end 143.51 100.9885) (width 0.5) (layer "F.Cu") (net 13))
 (segment (start 142.748 105.762) (end 142.845 105.665) (width 0.5) (layer "F.Cu") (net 13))
 (segment (start 142.845 105.665) (end 142.845 104.551) (width 0.5) (layer "F.Cu") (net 13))
 (segment (start 142.845 104.551) (end 143.256 104.14) (width 0.5) (layer "F.Cu") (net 13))
 (segment (start 135.128 126.238) (end 135.382 126.492) (width 0.5) (layer "F.Cu") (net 10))
 (segment (start 135.382 126.492) (end 135.382 128.016) (width 0.5) (layer "F.Cu") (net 10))
 (segment (start 135.128 115.062) (end 135.128 126.238) (width 0.5) (layer "F.Cu") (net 10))
 (segment (start 136.197 115.263) (end 136.197 126.291) (width 0.5) (layer "F.Cu") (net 11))
 (segment (start 136.398 115.062) (end 136.197 115.263) (width 0.5) (layer "F.Cu") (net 11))
 (segment (start 136.197 126.291) (end 137.922 128.016) (width 0.5) (layer "F.Cu") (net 11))
 (segment (start 138.684 121.468051) (end 138.176 121.976051) (width 0.5) (layer "F.Cu") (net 12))
 (segment (start 140.208 115.062) (end 140.208 116.075051) (width 0.5) (layer "F.Cu") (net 12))
 (segment (start 140.208 116.075051) (end 138.684 117.599051) (width 0.5) (layer "F.Cu") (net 12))
 (segment (start 138.176 121.976051) (end 138.176 125.73) (width 0.5) (layer "F.Cu") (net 12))
 (segment (start 138.176 125.73) (end 140.462 128.016) (width 0.5) (layer "F.Cu") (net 12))
 (segment (start 138.684 117.599051) (end 138.684 121.468051) (width 0.5) (layer "F.Cu") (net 12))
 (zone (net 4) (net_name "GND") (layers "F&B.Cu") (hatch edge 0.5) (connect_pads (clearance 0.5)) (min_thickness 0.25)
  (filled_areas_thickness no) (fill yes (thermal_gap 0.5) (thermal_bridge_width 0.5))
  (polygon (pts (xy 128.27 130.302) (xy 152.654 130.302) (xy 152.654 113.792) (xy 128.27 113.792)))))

